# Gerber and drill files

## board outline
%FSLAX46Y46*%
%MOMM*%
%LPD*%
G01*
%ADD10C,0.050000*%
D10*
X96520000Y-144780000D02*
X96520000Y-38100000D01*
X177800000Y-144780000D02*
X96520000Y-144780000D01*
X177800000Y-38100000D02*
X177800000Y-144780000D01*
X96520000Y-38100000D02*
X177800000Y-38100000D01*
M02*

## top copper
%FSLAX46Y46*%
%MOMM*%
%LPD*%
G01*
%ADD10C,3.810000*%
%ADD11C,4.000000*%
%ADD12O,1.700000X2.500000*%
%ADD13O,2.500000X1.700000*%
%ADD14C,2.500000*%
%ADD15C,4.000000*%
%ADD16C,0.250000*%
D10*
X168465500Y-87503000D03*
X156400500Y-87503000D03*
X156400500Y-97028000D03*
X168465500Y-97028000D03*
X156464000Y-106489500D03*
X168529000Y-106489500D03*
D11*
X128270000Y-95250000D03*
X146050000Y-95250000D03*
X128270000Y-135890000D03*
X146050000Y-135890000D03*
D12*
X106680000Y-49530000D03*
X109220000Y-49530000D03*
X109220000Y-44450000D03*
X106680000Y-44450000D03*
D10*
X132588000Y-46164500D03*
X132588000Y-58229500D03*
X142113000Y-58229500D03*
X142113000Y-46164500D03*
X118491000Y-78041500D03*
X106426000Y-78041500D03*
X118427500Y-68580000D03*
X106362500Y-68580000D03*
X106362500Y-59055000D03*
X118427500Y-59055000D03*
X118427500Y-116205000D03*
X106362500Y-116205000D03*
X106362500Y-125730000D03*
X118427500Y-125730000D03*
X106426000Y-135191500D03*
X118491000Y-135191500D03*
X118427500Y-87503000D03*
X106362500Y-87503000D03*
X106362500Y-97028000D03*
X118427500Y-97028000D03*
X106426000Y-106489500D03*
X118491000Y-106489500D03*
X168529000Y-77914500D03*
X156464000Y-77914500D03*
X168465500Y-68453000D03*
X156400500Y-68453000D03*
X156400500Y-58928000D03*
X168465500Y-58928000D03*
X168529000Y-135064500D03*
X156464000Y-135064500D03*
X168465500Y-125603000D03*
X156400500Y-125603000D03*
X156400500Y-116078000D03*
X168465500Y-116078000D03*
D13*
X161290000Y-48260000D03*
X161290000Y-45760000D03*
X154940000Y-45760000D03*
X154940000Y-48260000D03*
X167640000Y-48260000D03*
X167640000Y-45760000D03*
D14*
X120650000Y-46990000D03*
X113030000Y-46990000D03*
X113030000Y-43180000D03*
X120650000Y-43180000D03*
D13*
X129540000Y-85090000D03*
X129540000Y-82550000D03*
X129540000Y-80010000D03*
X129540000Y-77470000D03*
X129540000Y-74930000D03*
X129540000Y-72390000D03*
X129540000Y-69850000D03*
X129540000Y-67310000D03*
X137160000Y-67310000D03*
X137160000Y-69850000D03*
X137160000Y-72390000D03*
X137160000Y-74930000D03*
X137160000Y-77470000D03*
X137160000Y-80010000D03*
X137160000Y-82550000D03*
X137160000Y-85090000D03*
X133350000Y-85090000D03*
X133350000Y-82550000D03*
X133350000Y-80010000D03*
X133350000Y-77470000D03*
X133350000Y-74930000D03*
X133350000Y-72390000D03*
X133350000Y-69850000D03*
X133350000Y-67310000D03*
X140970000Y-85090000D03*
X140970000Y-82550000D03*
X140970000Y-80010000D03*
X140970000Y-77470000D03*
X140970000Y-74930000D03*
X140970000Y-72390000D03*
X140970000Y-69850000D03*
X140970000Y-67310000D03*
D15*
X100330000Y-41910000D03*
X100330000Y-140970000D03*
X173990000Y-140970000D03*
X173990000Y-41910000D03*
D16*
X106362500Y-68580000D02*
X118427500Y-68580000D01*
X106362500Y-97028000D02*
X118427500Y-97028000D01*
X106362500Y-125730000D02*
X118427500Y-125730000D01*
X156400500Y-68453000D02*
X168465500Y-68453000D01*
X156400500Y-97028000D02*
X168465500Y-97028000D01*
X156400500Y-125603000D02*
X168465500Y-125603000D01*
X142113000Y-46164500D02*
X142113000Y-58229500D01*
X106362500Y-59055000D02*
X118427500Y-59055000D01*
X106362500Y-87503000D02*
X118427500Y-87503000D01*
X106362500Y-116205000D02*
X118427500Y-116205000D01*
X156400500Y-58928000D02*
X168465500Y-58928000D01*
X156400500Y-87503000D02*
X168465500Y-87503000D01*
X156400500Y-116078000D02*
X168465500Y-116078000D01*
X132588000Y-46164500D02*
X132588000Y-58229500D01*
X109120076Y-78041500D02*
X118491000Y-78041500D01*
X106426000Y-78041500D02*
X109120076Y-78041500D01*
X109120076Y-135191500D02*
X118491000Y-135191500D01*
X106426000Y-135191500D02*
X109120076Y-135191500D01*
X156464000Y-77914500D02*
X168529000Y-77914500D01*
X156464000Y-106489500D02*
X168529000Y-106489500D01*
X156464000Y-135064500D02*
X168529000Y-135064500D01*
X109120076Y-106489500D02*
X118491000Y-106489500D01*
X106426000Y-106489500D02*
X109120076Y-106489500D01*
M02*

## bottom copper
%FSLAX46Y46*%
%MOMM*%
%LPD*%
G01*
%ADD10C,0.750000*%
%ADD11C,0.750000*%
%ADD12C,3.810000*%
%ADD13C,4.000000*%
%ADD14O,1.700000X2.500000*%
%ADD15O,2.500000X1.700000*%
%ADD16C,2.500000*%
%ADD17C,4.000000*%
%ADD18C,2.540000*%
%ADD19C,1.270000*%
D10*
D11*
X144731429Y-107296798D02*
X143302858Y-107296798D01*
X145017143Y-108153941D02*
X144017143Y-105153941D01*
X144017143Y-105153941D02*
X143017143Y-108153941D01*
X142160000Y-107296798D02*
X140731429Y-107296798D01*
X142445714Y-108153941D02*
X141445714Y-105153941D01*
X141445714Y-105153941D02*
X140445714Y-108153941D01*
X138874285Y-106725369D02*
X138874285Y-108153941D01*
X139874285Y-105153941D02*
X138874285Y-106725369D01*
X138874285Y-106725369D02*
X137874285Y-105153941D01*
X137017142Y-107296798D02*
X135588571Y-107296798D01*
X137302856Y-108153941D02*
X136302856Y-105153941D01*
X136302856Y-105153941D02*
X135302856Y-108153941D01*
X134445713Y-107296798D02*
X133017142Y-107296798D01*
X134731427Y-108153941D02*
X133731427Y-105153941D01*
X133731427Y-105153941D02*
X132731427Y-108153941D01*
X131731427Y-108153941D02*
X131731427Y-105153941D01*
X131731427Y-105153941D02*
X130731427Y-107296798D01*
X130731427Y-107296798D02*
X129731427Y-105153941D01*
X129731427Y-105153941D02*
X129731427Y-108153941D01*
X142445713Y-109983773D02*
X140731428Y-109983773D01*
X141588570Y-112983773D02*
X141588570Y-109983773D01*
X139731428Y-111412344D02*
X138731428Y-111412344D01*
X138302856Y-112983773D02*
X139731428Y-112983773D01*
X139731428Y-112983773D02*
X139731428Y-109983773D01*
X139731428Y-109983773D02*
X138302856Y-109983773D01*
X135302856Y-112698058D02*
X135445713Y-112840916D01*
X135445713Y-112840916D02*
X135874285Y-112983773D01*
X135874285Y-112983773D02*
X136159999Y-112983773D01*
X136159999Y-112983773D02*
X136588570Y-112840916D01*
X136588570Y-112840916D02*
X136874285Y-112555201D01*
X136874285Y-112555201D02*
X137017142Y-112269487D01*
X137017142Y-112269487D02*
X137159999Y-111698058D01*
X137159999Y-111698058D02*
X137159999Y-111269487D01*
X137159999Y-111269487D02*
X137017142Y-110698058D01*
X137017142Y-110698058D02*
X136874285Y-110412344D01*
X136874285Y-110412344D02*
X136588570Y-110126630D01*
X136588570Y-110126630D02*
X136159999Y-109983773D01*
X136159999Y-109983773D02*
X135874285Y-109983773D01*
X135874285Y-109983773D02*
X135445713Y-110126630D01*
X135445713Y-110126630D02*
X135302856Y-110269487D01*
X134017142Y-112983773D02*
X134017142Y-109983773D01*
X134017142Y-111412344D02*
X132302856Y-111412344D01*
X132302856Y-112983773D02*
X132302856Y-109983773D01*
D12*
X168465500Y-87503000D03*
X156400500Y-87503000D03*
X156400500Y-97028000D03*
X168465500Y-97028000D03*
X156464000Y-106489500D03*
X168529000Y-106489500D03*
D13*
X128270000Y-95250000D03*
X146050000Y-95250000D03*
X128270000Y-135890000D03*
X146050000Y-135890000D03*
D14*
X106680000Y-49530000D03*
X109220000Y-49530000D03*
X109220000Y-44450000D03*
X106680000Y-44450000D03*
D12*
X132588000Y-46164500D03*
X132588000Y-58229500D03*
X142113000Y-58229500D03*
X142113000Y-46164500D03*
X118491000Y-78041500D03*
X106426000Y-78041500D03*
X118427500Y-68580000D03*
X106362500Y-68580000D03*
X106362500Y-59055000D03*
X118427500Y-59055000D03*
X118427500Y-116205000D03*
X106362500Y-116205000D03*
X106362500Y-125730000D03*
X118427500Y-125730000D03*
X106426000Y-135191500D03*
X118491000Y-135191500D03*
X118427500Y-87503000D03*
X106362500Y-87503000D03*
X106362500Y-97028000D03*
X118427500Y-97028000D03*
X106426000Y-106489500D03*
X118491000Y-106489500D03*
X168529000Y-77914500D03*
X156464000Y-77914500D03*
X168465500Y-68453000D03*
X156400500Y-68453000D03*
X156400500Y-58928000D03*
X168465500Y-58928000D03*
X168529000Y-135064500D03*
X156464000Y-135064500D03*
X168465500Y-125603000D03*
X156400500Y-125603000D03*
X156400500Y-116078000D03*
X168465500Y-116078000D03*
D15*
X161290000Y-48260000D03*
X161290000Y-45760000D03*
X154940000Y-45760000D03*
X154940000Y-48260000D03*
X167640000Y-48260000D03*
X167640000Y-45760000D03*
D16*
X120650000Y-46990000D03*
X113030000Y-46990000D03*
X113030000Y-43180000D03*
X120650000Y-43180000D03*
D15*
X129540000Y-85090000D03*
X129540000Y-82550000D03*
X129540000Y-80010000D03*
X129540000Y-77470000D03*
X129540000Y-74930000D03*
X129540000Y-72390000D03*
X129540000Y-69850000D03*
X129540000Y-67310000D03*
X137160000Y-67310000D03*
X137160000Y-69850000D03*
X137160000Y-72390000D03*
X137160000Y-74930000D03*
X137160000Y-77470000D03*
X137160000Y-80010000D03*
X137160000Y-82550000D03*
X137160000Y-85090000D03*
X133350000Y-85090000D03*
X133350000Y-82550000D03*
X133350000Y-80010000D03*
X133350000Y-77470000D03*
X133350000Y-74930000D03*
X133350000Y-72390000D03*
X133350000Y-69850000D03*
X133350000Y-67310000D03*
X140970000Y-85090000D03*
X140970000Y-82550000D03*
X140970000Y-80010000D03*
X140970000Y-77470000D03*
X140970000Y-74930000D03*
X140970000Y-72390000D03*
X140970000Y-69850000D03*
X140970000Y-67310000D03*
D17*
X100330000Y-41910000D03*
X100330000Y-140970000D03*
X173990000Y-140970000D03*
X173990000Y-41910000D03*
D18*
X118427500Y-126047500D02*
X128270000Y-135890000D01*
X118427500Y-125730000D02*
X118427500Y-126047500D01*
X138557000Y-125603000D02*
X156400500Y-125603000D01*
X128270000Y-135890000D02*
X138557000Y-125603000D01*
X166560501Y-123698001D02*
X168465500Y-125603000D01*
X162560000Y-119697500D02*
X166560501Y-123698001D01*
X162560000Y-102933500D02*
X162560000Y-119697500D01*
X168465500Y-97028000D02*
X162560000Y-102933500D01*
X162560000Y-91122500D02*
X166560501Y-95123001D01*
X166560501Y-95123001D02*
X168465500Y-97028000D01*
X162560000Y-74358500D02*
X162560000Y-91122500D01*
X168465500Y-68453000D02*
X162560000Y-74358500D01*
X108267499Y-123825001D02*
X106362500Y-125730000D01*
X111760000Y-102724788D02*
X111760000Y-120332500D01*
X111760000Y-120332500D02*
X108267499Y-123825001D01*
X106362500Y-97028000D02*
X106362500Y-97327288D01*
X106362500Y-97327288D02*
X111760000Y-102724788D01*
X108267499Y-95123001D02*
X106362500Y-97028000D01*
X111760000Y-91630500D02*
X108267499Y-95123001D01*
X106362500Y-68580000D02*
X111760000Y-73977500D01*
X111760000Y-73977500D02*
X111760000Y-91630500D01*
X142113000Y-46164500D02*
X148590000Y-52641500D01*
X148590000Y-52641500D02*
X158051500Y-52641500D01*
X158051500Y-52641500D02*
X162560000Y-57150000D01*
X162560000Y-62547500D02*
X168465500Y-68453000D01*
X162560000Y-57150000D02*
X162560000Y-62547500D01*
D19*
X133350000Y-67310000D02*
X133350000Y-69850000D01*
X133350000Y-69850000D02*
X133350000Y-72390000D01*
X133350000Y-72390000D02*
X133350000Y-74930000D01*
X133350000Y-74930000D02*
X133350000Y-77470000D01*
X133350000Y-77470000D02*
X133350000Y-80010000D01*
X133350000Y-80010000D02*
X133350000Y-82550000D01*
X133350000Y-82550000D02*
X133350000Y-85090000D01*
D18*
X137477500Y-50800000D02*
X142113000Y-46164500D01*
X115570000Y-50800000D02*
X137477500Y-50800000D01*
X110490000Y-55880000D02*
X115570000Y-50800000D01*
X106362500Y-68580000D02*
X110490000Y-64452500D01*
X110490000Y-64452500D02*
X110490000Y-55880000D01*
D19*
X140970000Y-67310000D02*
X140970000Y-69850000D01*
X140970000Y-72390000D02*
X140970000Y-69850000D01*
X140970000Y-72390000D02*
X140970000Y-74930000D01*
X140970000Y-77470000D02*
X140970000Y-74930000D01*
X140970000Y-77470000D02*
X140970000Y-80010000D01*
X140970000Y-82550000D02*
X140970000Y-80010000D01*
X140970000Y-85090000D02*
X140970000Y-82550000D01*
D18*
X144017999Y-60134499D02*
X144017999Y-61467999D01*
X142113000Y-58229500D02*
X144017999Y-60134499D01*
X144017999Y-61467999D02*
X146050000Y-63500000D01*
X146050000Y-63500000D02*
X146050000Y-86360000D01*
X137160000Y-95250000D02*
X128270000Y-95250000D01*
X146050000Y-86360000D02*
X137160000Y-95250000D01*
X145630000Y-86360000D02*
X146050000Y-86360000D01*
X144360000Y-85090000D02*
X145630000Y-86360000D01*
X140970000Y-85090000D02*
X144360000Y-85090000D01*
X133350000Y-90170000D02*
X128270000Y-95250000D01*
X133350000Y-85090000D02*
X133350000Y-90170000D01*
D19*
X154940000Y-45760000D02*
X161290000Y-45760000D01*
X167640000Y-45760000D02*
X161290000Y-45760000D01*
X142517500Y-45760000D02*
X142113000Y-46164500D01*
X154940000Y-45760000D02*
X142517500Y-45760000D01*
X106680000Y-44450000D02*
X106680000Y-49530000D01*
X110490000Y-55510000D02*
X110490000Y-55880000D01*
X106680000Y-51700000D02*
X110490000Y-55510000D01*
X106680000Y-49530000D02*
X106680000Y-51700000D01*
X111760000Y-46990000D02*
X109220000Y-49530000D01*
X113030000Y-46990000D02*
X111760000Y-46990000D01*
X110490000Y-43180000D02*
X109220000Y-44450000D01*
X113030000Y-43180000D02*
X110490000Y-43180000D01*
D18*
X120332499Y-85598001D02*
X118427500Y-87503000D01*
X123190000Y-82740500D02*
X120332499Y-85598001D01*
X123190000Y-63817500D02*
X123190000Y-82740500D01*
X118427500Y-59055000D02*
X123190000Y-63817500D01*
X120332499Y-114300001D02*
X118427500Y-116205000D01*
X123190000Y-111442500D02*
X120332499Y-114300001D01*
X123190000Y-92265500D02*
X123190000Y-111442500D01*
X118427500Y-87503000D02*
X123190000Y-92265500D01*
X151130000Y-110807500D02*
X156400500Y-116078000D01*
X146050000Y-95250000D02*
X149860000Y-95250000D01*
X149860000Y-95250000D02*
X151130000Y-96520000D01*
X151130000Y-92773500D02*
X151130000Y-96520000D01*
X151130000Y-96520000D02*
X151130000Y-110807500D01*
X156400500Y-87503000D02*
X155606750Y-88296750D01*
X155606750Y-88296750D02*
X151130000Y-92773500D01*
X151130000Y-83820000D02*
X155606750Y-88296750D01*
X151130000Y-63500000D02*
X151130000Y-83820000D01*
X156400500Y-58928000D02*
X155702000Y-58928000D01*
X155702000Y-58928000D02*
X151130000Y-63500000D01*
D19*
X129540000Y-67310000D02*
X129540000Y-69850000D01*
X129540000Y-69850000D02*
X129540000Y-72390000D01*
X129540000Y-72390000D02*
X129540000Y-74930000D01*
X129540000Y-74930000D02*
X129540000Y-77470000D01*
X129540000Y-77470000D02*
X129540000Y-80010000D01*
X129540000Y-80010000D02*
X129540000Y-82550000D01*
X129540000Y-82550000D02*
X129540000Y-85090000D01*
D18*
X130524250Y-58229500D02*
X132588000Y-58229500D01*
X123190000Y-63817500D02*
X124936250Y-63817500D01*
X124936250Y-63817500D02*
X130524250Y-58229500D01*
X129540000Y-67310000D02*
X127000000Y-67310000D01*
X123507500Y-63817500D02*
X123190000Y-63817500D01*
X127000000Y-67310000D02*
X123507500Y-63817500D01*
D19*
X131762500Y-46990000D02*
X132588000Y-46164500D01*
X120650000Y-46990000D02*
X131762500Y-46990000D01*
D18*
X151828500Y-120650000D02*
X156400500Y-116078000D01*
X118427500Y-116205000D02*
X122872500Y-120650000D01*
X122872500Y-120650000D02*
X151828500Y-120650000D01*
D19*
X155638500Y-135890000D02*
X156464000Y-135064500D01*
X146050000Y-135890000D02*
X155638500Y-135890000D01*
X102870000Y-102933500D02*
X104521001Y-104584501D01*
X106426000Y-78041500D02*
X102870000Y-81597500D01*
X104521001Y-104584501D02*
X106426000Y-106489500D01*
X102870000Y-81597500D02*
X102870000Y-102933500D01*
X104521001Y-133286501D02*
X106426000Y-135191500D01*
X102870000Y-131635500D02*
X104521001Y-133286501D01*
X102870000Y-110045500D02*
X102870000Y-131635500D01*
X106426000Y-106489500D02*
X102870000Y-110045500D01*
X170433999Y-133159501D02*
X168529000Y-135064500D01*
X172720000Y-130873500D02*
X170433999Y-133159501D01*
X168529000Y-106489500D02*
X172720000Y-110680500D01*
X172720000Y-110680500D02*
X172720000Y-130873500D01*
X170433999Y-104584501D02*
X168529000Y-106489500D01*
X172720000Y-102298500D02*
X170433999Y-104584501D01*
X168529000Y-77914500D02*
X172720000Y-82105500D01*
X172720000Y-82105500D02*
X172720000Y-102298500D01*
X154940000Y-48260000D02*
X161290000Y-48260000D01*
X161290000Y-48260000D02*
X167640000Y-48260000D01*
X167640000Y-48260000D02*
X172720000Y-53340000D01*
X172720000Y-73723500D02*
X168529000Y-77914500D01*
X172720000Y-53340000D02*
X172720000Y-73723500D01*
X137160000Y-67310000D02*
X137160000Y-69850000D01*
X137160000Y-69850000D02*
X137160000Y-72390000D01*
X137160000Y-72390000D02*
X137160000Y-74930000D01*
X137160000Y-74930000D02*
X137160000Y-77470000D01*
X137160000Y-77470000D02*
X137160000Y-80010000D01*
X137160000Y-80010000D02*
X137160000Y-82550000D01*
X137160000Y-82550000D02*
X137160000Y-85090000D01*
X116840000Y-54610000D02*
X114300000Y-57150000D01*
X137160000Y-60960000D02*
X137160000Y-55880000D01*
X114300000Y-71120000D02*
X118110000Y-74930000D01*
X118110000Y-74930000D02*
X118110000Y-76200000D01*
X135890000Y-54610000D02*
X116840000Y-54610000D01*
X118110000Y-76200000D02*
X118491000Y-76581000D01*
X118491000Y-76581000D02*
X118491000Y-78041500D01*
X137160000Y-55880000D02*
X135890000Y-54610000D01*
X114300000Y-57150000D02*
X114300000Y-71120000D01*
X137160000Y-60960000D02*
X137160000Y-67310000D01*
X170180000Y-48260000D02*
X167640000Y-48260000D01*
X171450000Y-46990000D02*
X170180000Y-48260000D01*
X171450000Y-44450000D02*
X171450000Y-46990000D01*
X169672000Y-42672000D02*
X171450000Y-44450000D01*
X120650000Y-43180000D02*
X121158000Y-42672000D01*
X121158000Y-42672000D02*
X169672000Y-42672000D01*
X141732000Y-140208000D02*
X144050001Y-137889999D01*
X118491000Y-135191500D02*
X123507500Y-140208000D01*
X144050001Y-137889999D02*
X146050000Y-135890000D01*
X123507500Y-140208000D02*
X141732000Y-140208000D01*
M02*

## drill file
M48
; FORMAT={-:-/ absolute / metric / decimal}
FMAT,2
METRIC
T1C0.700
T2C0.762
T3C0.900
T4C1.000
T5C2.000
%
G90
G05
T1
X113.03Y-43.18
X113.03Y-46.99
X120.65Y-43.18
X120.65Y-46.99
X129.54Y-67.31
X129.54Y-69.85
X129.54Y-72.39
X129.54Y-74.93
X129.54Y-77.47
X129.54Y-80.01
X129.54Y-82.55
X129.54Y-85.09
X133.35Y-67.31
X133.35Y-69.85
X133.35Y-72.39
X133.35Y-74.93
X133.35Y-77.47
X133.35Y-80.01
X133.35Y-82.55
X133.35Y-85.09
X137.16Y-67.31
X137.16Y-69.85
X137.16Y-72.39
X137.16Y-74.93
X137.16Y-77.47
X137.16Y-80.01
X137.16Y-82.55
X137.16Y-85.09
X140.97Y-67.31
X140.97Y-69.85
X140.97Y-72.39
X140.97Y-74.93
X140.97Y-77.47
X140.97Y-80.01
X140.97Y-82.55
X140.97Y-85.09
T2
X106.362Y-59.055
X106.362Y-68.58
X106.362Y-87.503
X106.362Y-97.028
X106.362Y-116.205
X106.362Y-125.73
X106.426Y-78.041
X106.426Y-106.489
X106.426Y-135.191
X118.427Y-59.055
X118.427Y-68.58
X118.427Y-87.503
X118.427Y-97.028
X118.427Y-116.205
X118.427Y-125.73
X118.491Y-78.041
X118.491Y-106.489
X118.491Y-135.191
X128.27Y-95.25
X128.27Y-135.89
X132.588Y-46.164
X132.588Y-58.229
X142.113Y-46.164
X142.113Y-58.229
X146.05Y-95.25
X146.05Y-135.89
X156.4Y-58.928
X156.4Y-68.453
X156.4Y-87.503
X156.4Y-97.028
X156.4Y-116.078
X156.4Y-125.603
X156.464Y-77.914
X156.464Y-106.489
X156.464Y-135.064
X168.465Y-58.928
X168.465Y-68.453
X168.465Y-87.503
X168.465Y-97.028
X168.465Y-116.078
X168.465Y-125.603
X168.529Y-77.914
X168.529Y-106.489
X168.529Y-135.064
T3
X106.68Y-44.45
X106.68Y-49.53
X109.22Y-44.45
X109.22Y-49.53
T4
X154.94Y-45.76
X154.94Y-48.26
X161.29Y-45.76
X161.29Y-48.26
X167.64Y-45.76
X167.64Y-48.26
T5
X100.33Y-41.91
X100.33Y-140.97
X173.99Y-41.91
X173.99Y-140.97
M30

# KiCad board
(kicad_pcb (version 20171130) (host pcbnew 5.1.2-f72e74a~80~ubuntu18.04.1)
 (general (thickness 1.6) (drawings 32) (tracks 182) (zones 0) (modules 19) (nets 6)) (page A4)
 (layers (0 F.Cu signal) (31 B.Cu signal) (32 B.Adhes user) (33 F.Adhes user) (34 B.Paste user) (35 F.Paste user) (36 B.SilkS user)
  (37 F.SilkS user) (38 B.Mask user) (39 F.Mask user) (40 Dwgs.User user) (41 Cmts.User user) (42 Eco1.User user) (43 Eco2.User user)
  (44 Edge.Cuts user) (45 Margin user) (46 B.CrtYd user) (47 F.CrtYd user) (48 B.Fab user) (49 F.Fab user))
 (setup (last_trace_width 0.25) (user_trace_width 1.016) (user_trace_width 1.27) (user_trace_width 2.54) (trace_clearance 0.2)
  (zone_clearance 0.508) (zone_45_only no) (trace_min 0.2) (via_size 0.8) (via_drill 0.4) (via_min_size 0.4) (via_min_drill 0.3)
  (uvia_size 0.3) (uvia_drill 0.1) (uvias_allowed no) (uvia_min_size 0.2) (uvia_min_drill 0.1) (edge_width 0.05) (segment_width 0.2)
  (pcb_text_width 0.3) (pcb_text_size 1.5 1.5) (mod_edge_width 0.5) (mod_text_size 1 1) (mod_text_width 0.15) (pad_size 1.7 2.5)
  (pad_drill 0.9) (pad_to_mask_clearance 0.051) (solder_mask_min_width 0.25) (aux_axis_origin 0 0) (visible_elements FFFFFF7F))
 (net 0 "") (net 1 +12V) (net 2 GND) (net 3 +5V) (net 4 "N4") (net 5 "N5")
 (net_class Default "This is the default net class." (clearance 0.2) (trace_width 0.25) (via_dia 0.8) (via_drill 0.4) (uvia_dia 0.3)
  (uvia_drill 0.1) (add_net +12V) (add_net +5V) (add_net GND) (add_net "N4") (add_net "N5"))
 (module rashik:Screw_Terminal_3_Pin (layer F.Cu) (at 162.56 97.155 270)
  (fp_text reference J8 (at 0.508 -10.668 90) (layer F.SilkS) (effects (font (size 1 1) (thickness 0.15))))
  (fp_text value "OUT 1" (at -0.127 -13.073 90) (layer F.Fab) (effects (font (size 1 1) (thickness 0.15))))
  (pad 1 thru_hole circle (at -9.652 -5.9055 270) (size 3.81 3.81) (drill 0.762) (layers *.Cu *.Mask) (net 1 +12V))
  (pad 1 thru_hole circle (at -9.652 6.1595 270) (size 3.81 3.81) (drill 0.762) (layers *.Cu *.Mask) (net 1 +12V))
  (pad 2 thru_hole circle (at -0.127 6.1595 270) (size 3.81 3.81) (drill 0.762) (layers *.Cu *.Mask) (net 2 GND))
  (pad 2 thru_hole circle (at -0.127 -5.9055 270) (size 3.81 3.81) (drill 0.762) (layers *.Cu *.Mask) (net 2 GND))
  (pad 3 thru_hole circle (at 9.3345 6.096 270) (size 3.81 3.81) (drill 0.762) (layers *.Cu *.Mask) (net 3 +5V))
  (pad 3 thru_hole circle (at 9.3345 -5.969 270) (size 3.81 3.81) (drill 0.762) (layers *.Cu *.Mask) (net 3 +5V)))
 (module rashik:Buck (layer F.Cu) (at 135.89 115.57)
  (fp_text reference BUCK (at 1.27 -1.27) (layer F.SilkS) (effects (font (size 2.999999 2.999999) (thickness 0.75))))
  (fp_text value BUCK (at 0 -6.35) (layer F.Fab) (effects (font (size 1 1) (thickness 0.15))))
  (pad 1 thru_hole circle (at -7.62 -20.32) (size 4 4) (drill 0.762) (layers *.Cu *.Mask) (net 2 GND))
  (pad 2 thru_hole circle (at 10.16 -20.32) (size 4 4) (drill 0.762) (layers *.Cu *.Mask) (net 1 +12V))
  (pad 3 thru_hole circle (at -7.62 20.32) (size 4 4) (drill 0.762) (layers *.Cu *.Mask) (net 2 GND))
  (pad 4 thru_hole circle (at 10.16 20.32) (size 4 4) (drill 0.762) (layers *.Cu *.Mask) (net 3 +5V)))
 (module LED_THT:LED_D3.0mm (layer F.Cu) (at 106.68 49.53)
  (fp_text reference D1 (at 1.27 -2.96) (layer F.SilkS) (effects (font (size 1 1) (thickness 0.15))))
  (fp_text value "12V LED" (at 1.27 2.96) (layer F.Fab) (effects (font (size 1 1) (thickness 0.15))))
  (pad 1 thru_hole oval (at 0 0) (size 1.7 2.5) (drill 0.9) (layers *.Cu *.Mask) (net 2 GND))
  (pad 2 thru_hole oval (at 2.54 0) (size 1.7 2.5) (drill 0.9) (layers *.Cu *.Mask) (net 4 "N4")))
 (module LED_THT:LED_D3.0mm (layer F.Cu) (at 106.68 44.45)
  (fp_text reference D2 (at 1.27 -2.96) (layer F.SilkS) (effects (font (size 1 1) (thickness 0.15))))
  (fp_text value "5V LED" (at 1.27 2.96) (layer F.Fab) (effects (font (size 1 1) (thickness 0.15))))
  (pad 2 thru_hole oval (at 2.54 0) (size 1.7 2.5) (drill 0.9) (layers *.Cu *.Mask) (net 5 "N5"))
  (pad 1 thru_hole oval (at 0 0) (size 1.7 2.5) (drill 0.9) (layers *.Cu *.Mask) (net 2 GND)))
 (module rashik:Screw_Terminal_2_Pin (layer F.Cu) (at 142.24 52.07)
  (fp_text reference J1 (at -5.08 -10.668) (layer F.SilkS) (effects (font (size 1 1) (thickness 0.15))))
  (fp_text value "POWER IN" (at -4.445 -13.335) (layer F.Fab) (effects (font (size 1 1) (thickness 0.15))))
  (pad 1 thru_hole circle (at -9.652 -5.9055) (size 3.81 3.81) (drill 0.762) (layers *.Cu *.Mask) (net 1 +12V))
  (pad 1 thru_hole circle (at -9.652 6.1595) (size 3.81 3.81) (drill 0.762) (layers *.Cu *.Mask) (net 1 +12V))
  (pad 2 thru_hole circle (at -0.127 6.1595) (size 3.81 3.81) (drill 0.762) (layers *.Cu *.Mask) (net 2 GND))
  (pad 2 thru_hole circle (at -0.127 -5.9055) (size 3.81 3.81) (drill 0.762) (layers *.Cu *.Mask) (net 2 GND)))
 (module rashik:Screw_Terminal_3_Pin (layer F.Cu) (at 112.522 68.707 270)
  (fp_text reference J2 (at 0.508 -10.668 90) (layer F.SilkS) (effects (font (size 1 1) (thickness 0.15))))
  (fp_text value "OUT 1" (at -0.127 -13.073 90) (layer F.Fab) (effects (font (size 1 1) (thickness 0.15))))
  (pad 3 thru_hole circle (at 9.3345 -5.969 270) (size 3.81 3.81) (drill 0.762) (layers *.Cu *.Mask) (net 3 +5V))
  (pad 3 thru_hole circle (at 9.3345 6.096 270) (size 3.81 3.81) (drill 0.762) (layers *.Cu *.Mask) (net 3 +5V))
  (pad 2 thru_hole circle (at -0.127 -5.9055 270) (size 3.81 3.81) (drill 0.762) (layers *.Cu *.Mask) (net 2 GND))
  (pad 2 thru_hole circle (at -0.127 6.1595 270) (size 3.81 3.81) (drill 0.762) (layers *.Cu *.Mask) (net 2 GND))
  (pad 1 thru_hole circle (at -9.652 6.1595 270) (size 3.81 3.81) (drill 0.762) (layers *.Cu *.Mask) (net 1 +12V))
  (pad 1 thru_hole circle (at -9.652 -5.9055 270) (size 3.81 3.81) (drill 0.762) (layers *.Cu *.Mask) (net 1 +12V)))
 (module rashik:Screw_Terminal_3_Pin (layer F.Cu) (at 112.522 125.857 270)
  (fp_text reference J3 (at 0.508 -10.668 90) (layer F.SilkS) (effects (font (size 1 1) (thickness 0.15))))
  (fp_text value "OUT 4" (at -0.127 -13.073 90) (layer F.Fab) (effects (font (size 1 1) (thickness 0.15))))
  (pad 1 thru_hole circle (at -9.652 -5.9055 270) (size 3.81 3.81) (drill 0.762) (layers *.Cu *.Mask) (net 1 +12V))
  (pad 1 thru_hole circle (at -9.652 6.1595 270) (size 3.81 3.81) (drill 0.762) (layers *.Cu *.Mask) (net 1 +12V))
  (pad 2 thru_hole circle (at -0.127 6.1595 270) (size 3.81 3.81) (drill 0.762) (layers *.Cu *.Mask) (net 2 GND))
  (pad 2 thru_hole circle (at -0.127 -5.9055 270) (size 3.81 3.81) (drill 0.762) (layers *.Cu *.Mask) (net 2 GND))
  (pad 3 thru_hole circle (at 9.3345 6.096 270) (size 3.81 3.81) (drill 0.762) (layers *.Cu *.Mask) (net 3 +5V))
  (pad 3 thru_hole circle (at 9.3345 -5.969 270) (size 3.81 3.81) (drill 0.762) (layers *.Cu *.Mask) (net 3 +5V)))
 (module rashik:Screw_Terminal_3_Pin (layer F.Cu) (at 112.522 97.155 270)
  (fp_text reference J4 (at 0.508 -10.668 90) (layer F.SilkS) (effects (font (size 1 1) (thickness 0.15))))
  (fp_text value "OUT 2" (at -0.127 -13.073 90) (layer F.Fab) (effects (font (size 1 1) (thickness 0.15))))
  (pad 1 thru_hole circle (at -9.652 -5.9055 270) (size 3.81 3.81) (drill 0.762) (layers *.Cu *.Mask) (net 1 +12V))
  (pad 1 thru_hole circle (at -9.652 6.1595 270) (size 3.81 3.81) (drill 0.762) (layers *.Cu *.Mask) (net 1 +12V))
  (pad 2 thru_hole circle (at -0.127 6.1595 270) (size 3.81 3.81) (drill 0.762) (layers *.Cu *.Mask) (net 2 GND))
  (pad 2 thru_hole circle (at -0.127 -5.9055 270) (size 3.81 3.81) (drill 0.762) (layers *.Cu *.Mask) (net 2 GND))
  (pad 3 thru_hole circle (at 9.3345 6.096 270) (size 3.81 3.81) (drill 0.762) (layers *.Cu *.Mask) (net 3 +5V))
  (pad 3 thru_hole circle (at 9.3345 -5.969 270) (size 3.81 3.81) (drill 0.762) (layers *.Cu *.Mask) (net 3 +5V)))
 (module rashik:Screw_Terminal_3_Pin (layer F.Cu) (at 162.56 68.58 270)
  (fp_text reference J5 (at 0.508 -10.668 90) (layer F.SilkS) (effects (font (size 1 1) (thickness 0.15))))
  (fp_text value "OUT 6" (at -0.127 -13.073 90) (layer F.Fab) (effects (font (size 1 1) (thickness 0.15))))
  (pad 3 thru_hole circle (at 9.3345 -5.969 270) (size 3.81 3.81) (drill 0.762) (layers *.Cu *.Mask) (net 3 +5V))
  (pad 3 thru_hole circle (at 9.3345 6.096 270) (size 3.81 3.81) (drill 0.762) (layers *.Cu *.Mask) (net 3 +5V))
  (pad 2 thru_hole circle (at -0.127 -5.9055 270) (size 3.81 3.81) (drill 0.762) (layers *.Cu *.Mask) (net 2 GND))
  (pad 2 thru_hole circle (at -0.127 6.1595 270) (size 3.81 3.81) (drill 0.762) (layers *.Cu *.Mask) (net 2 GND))
  (pad 1 thru_hole circle (at -9.652 6.1595 270) (size 3.81 3.81) (drill 0.762) (layers *.Cu *.Mask) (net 1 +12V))
  (pad 1 thru_hole circle (at -9.652 -5.9055 270) (size 3.81 3.81) (drill 0.762) (layers *.Cu *.Mask) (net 1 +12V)))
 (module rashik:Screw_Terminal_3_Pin (layer F.Cu) (at 162.56 125.73 270)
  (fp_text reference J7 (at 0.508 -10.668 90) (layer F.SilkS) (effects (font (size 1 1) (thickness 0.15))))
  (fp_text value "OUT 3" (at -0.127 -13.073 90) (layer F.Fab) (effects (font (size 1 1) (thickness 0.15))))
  (pad 3 thru_hole circle (at 9.3345 -5.969 270) (size 3.81 3.81) (drill 0.762) (layers *.Cu *.Mask) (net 3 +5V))
  (pad 3 thru_hole circle (at 9.3345 6.096 270) (size 3.81 3.81) (drill 0.762) (layers *.Cu *.Mask) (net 3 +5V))
  (pad 2 thru_hole circle (at -0.127 -5.9055 270) (size 3.81 3.81) (drill 0.762) (layers *.Cu *.Mask) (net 2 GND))
  (pad 2 thru_hole circle (at -0.127 6.1595 270) (size 3.81 3.81) (drill 0.762) (layers *.Cu *.Mask) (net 2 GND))
  (pad 1 thru_hole circle (at -9.652 6.1595 270) (size 3.81 3.81) (drill 0.762) (layers *.Cu *.Mask) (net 1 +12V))
  (pad 1 thru_hole circle (at -9.652 -5.9055 270) (size 3.81 3.81) (drill 0.762) (layers *.Cu *.Mask) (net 1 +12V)))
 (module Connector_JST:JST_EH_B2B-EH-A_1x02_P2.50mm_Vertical (layer F.Cu) (at 161.29 48.26 90)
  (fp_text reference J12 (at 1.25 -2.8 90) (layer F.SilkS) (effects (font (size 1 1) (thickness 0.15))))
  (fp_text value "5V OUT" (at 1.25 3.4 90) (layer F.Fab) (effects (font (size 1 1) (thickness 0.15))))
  (pad 1 thru_hole oval (at 0 0 90) (size 1.7 2.5) (drill 1) (layers *.Cu *.Mask) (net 3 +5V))
  (pad 2 thru_hole oval (at 2.5 0 90) (size 1.7 2.5) (drill 1) (layers *.Cu *.Mask) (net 2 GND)))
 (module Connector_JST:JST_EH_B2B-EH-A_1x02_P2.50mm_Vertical (layer F.Cu) (at 154.94 48.26 90)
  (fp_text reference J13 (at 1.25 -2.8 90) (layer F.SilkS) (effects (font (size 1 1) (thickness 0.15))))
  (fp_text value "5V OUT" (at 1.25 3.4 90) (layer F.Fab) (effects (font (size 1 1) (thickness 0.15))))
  (pad 2 thru_hole oval (at 2.5 0 90) (size 1.7 2.5) (drill 1) (layers *.Cu *.Mask) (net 2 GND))
  (pad 1 thru_hole oval (at 0 0 90) (size 1.7 2.5) (drill 1) (layers *.Cu *.Mask) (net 3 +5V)))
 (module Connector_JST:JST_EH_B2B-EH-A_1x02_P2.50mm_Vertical (layer F.Cu) (at 167.64 48.26 90)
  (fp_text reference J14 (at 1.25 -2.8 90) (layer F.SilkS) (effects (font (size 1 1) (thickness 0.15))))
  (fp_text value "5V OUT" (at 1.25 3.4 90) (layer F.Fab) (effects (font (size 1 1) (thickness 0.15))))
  (pad 1 thru_hole oval (at 0 0 90) (size 1.7 2.5) (drill 1) (layers *.Cu *.Mask) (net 3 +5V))
  (pad 2 thru_hole oval (at 2.5 0 90) (size 1.7 2.5) (drill 1) (layers *.Cu *.Mask) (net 2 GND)))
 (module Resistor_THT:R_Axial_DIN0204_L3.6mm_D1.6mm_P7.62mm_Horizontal (layer F.Cu) (at 113.03 46.99)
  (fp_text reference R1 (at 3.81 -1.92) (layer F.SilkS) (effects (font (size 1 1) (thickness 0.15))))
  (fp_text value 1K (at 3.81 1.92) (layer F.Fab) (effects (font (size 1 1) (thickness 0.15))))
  (pad 2 thru_hole circle (at 7.62 0) (size 2.5 2.5) (drill 0.7) (layers *.Cu *.Mask) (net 1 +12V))
  (pad 1 thru_hole circle (at 0 0) (size 2.5 2.5) (drill 0.7) (layers *.Cu *.Mask) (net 4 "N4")))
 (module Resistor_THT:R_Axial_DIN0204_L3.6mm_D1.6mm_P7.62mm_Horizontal (layer F.Cu) (at 113.03 43.18)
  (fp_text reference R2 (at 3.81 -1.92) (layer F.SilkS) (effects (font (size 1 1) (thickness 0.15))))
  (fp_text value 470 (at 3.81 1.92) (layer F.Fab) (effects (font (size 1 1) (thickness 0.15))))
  (pad 1 thru_hole circle (at 0 0) (size 2.5 2.5) (drill 0.7) (layers *.Cu *.Mask) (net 5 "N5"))
  (pad 2 thru_hole circle (at 7.62 0) (size 2.5 2.5) (drill 0.7) (layers *.Cu *.Mask) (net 3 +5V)))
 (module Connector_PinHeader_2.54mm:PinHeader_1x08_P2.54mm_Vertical (layer F.Cu) (at 129.54 85.09 180)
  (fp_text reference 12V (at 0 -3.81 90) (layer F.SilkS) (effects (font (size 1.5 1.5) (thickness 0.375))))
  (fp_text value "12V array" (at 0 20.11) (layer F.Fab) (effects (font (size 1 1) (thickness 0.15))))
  (pad 1 thru_hole oval (at 0 0 180) (size 2.5 1.7) (drill 0.7) (layers *.Cu *.Mask) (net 1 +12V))
  (pad 2 thru_hole oval (at 0 2.54 180) (size 2.5 1.7) (drill 0.7) (layers *.Cu *.Mask) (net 1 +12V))
  (pad 3 thru_hole oval (at 0 5.08 180) (size 2.5 1.7) (drill 0.7) (layers *.Cu *.Mask) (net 1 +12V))
  (pad 4 thru_hole oval (at 0 7.62 180) (size 2.5 1.7) (drill 0.7) (layers *.Cu *.Mask) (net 1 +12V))
  (pad 5 thru_hole oval (at 0 10.16 180) (size 2.5 1.7) (drill 0.7) (layers *.Cu *.Mask) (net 1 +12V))
  (pad 6 thru_hole oval (at 0 12.7 180) (size 2.5 1.7) (drill 0.7) (layers *.Cu *.Mask) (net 1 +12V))
  (pad 7 thru_hole oval (at 0 15.24 180) (size 2.5 1.7) (drill 0.7) (layers *.Cu *.Mask) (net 1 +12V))
  (pad 8 thru_hole oval (at 0 17.78 180) (size 2.5 1.7) (drill 0.7) (layers *.Cu *.Mask) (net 1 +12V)))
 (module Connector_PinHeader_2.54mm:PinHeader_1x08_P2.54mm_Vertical (layer F.Cu) (at 137.16 85.09 180)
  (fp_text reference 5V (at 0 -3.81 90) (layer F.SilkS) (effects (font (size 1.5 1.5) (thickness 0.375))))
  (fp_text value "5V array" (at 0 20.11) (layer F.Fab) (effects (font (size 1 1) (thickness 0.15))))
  (pad 8 thru_hole oval (at 0 17.78 180) (size 2.5 1.7) (drill 0.7) (layers *.Cu *.Mask) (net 3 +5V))
  (pad 7 thru_hole oval (at 0 15.24 180) (size 2.5 1.7) (drill 0.7) (layers *.Cu *.Mask) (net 3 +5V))
  (pad 6 thru_hole oval (at 0 12.7 180) (size 2.5 1.7) (drill 0.7) (layers *.Cu *.Mask) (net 3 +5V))
  (pad 5 thru_hole oval (at 0 10.16 180) (size 2.5 1.7) (drill 0.7) (layers *.Cu *.Mask) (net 3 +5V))
  (pad 4 thru_hole oval (at 0 7.62 180) (size 2.5 1.7) (drill 0.7) (layers *.Cu *.Mask) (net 3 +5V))
  (pad 3 thru_hole oval (at 0 5.08 180) (size 2.5 1.7) (drill 0.7) (layers *.Cu *.Mask) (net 3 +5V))
  (pad 2 thru_hole oval (at 0 2.54 180) (size 2.5 1.7) (drill 0.7) (layers *.Cu *.Mask) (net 3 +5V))
  (pad 1 thru_hole oval (at 0 0 180) (size 2.5 1.7) (drill 0.7) (layers *.Cu *.Mask) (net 3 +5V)))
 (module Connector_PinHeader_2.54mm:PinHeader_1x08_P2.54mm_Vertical (layer F.Cu) (at 133.35 85.09 180)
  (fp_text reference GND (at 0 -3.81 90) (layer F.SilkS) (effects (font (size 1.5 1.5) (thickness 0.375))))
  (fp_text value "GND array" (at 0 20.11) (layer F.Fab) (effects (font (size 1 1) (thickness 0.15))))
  (pad 1 thru_hole oval (at 0 0 180) (size 2.5 1.7) (drill 0.7) (layers *.Cu *.Mask) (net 2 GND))
  (pad 2 thru_hole oval (at 0 2.54 180) (size 2.5 1.7) (drill 0.7) (layers *.Cu *.Mask) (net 2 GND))
  (pad 3 thru_hole oval (at 0 5.08 180) (size 2.5 1.7) (drill 0.7) (layers *.Cu *.Mask) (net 2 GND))
  (pad 4 thru_hole oval (at 0 7.62 180) (size 2.5 1.7) (drill 0.7) (layers *.Cu *.Mask) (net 2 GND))
  (pad 5 thru_hole oval (at 0 10.16 180) (size 2.5 1.7) (drill 0.7) (layers *.Cu *.Mask) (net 2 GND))
  (pad 6 thru_hole oval (at 0 12.7 180) (size 2.5 1.7) (drill 0.7) (layers *.Cu *.Mask) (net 2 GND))
  (pad 7 thru_hole oval (at 0 15.24 180) (size 2.5 1.7) (drill 0.7) (layers *.Cu *.Mask) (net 2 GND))
  (pad 8 thru_hole oval (at 0 17.78 180) (size 2.5 1.7) (drill 0.7) (layers *.Cu *.Mask) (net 2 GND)))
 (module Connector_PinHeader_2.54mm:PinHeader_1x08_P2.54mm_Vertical (layer F.Cu) (at 140.97 85.09 180)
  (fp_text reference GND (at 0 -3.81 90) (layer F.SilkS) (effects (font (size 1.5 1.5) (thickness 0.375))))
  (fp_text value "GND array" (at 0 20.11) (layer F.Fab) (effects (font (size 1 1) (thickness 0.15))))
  (pad 1 thru_hole oval (at 0 0 180) (size 2.5 1.7) (drill 0.7) (layers *.Cu *.Mask) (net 2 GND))
  (pad 2 thru_hole oval (at 0 2.54 180) (size 2.5 1.7) (drill 0.7) (layers *.Cu *.Mask) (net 2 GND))
  (pad 3 thru_hole oval (at 0 5.08 180) (size 2.5 1.7) (drill 0.7) (layers *.Cu *.Mask) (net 2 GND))
  (pad 4 thru_hole oval (at 0 7.62 180) (size 2.5 1.7) (drill 0.7) (layers *.Cu *.Mask) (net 2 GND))
  (pad 5 thru_hole oval (at 0 10.16 180) (size 2.5 1.7) (drill 0.7) (layers *.Cu *.Mask) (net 2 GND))
  (pad 6 thru_hole oval (at 0 12.7 180) (size 2.5 1.7) (drill 0.7) (layers *.Cu *.Mask) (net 2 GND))
  (pad 7 thru_hole oval (at 0 15.24 180) (size 2.5 1.7) (drill 0.7) (layers *.Cu *.Mask) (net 2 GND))
  (pad 8 thru_hole oval (at 0 17.78 180) (size 2.5 1.7) (drill 0.7) (layers *.Cu *.Mask) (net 2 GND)))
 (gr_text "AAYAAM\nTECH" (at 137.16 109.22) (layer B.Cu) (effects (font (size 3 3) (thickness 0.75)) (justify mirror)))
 (gr_line (start 96.52 144.78) (end 96.52 38.1) (layer Edge.Cuts) (width 0.05))
 (gr_line (start 177.8 144.78) (end 96.52 144.78) (layer Edge.Cuts) (width 0.05))
 (gr_line (start 177.8 38.1) (end 177.8 144.78) (layer Edge.Cuts) (width 0.05))
 (gr_line (start 96.52 38.1) (end 177.8 38.1) (layer Edge.Cuts) (width 0.05))
 (via (at 100.33 41.91) (size 4) (drill 2) (layers F.Cu B.Cu) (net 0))
 (via (at 100.33 140.97) (size 4) (drill 2) (layers F.Cu B.Cu) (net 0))
 (via (at 173.99 140.97) (size 4) (drill 2) (layers F.Cu B.Cu) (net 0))
 (via (at 173.99 41.91) (size 4) (drill 2) (layers F.Cu B.Cu) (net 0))
 (segment (start 118.4275 126.0475) (end 128.27 135.89) (width 2.54) (layer B.Cu) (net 2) (status 30))
 (segment (start 118.4275 125.73) (end 118.4275 126.0475) (width 2.54) (layer B.Cu) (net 2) (status 30))
 (segment (start 138.557 125.603) (end 156.4005 125.603) (width 2.54) (layer B.Cu) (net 2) (status 20))
 (segment (start 128.27 135.89) (end 138.557 125.603) (width 2.54) (layer B.Cu) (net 2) (status 10))
 (segment (start 166.560501 123.698001) (end 168.4655 125.603) (width 2.54) (layer B.Cu) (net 2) (status 20))
 (segment (start 162.56 119.6975) (end 166.560501 123.698001) (width 2.54) (layer B.Cu) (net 2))
 (segment (start 162.56 102.9335) (end 162.56 119.6975) (width 2.54) (layer B.Cu) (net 2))
 (segment (start 168.4655 97.028) (end 162.56 102.9335) (width 2.54) (layer B.Cu) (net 2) (status 10))
 (segment (start 162.56 91.1225) (end 166.560501 95.123001) (width 2.54) (layer B.Cu) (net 2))
 (segment (start 166.560501 95.123001) (end 168.4655 97.028) (width 2.54) (layer B.Cu) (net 2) (status 20))
 (segment (start 162.56 74.3585) (end 162.56 91.1225) (width 2.54) (layer B.Cu) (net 2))
 (segment (start 168.4655 68.453) (end 162.56 74.3585) (width 2.54) (layer B.Cu) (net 2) (status 10))
 (segment (start 108.267499 123.825001) (end 106.3625 125.73) (width 2.54) (layer B.Cu) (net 2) (status 20))
 (segment (start 111.76 102.724788) (end 111.76 120.3325) (width 2.54) (layer B.Cu) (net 2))
 (segment (start 111.76 120.3325) (end 108.267499 123.825001) (width 2.54) (layer B.Cu) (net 2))
 (segment (start 106.3625 97.028) (end 106.3625 97.327288) (width 2.54) (layer B.Cu) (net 2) (status 30))
 (segment (start 106.3625 97.327288) (end 111.76 102.724788) (width 2.54) (layer B.Cu) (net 2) (status 10))
 (segment (start 108.267499 95.123001) (end 106.3625 97.028) (width 2.54) (layer B.Cu) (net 2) (status 20))
 (segment (start 111.76 91.6305) (end 108.267499 95.123001) (width 2.54) (layer B.Cu) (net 2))
 (segment (start 106.3625 68.58) (end 111.76 73.9775) (width 2.54) (layer B.Cu) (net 2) (status 10))
 (segment (start 111.76 73.9775) (end 111.76 91.6305) (width 2.54) (layer B.Cu) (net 2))
 (segment (start 142.113 46.1645) (end 148.59 52.6415) (width 2.54) (layer B.Cu) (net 2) (status 10))
 (segment (start 148.59 52.6415) (end 158.0515 52.6415) (width 2.54) (layer B.Cu) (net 2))
 (segment (start 158.0515 52.6415) (end 162.56 57.15) (width 2.54) (layer B.Cu) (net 2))
 (segment (start 162.56 62.5475) (end 168.4655 68.453) (width 2.54) (layer B.Cu) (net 2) (status 20))
 (segment (start 162.56 57.15) (end 162.56 62.5475) (width 2.54) (layer B.Cu) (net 2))
 (segment (start 133.35 67.31) (end 133.35 69.85) (width 1.27) (layer B.Cu) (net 2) (status 30))
 (segment (start 133.35 69.85) (end 133.35 72.39) (width 1.27) (layer B.Cu) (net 2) (status 30))
 (segment (start 133.35 72.39) (end 133.35 74.93) (width 1.27) (layer B.Cu) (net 2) (status 30))
 (segment (start 133.35 74.93) (end 133.35 77.47) (width 1.27) (layer B.Cu) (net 2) (status 30))
 (segment (start 133.35 77.47) (end 133.35 80.01) (width 1.27) (layer B.Cu) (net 2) (status 30))
 (segment (start 133.35 80.01) (end 133.35 82.55) (width 1.27) (layer B.Cu) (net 2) (status 30))
 (segment (start 133.35 82.55) (end 133.35 85.09) (width 1.27) (layer B.Cu) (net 2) (status 30))
 (segment (start 137.4775 50.8) (end 142.113 46.1645) (width 2.54) (layer B.Cu) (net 2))
 (segment (start 115.57 50.8) (end 137.4775 50.8) (width 2.54) (layer B.Cu) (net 2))
 (segment (start 110.49 55.88) (end 115.57 50.8) (width 2.54) (layer B.Cu) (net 2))
 (segment (start 106.3625 68.58) (end 110.49 64.4525) (width 2.54) (layer B.Cu) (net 2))
 (segment (start 110.49 64.4525) (end 110.49 55.88) (width 2.54) (layer B.Cu) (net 2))
 (segment (start 140.97 67.31) (end 140.97 69.85) (width 1.27) (layer B.Cu) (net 2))
 (segment (start 140.97 72.39) (end 140.97 69.85) (width 1.27) (layer B.Cu) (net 2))
 (segment (start 140.97 72.39) (end 140.97 74.93) (width 1.27) (layer B.Cu) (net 2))
 (segment (start 140.97 77.47) (end 140.97 74.93) (width 1.27) (layer B.Cu) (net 2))
 (segment (start 140.97 77.47) (end 140.97 80.01) (width 1.27) (layer B.Cu) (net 2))
 (segment (start 140.97 82.55) (end 140.97 80.01) (width 1.27) (layer B.Cu) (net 2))
 (segment (start 140.97 85.09) (end 140.97 82.55) (width 1.27) (layer B.Cu) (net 2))
 (segment (start 106.3625 68.58) (end 118.4275 68.58) (width 0.25) (layer F.Cu) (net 2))
 (segment (start 106.3625 97.028) (end 118.4275 97.028) (width 0.25) (layer F.Cu) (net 2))
 (segment (start 106.3625 125.73) (end 118.4275 125.73) (width 0.25) (layer F.Cu) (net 2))
 (segment (start 156.4005 68.453) (end 168.4655 68.453) (width 0.25) (layer F.Cu) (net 2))
 (segment (start 156.4005 97.028) (end 168.4655 97.028) (width 0.25) (layer F.Cu) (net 2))
 (segment (start 156.4005 125.603) (end 168.4655 125.603) (width 0.25) (layer F.Cu) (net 2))
 (segment (start 144.017999 60.134499) (end 144.017999 61.467999) (width 2.54) (layer B.Cu) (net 2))
 (segment (start 142.113 58.2295) (end 144.017999 60.134499) (width 2.54) (layer B.Cu) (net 2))
 (segment (start 144.017999 61.467999) (end 146.05 63.5) (width 2.54) (layer B.Cu) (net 2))
 (segment (start 146.05 63.5) (end 146.05 86.36) (width 2.54) (layer B.Cu) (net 2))
 (segment (start 137.16 95.25) (end 128.27 95.25) (width 2.54) (layer B.Cu) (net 2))
 (segment (start 146.05 86.36) (end 137.16 95.25) (width 2.54) (layer B.Cu) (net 2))
 (segment (start 145.63 86.36) (end 146.05 86.36) (width 2.54) (layer B.Cu) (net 2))
 (segment (start 144.36 85.09) (end 145.63 86.36) (width 2.54) (layer B.Cu) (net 2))
 (segment (start 140.97 85.09) (end 144.36 85.09) (width 2.54) (layer B.Cu) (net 2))
 (segment (start 133.35 90.17) (end 128.27 95.25) (width 2.54) (layer B.Cu) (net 2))
 (segment (start 133.35 85.09) (end 133.35 90.17) (width 2.54) (layer B.Cu) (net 2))
 (segment (start 154.94 45.76) (end 161.29 45.76) (width 1.27) (layer B.Cu) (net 2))
 (segment (start 167.64 45.76) (end 161.29 45.76) (width 1.27) (layer B.Cu) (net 2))
 (segment (start 142.5175 45.76) (end 142.113 46.1645) (width 1.27) (layer B.Cu) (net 2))
 (segment (start 154.94 45.76) (end 142.5175 45.76) (width 1.27) (layer B.Cu) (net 2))
 (segment (start 106.68 44.45) (end 106.68 49.53) (width 1.27) (layer B.Cu) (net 2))
 (segment (start 110.49 55.51) (end 110.49 55.88) (width 1.27) (layer B.Cu) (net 2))
 (segment (start 106.68 51.7) (end 110.49 55.51) (width 1.27) (layer B.Cu) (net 2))
 (segment (start 106.68 49.53) (end 106.68 51.7) (width 1.27) (layer B.Cu) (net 2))
 (segment (start 142.113 46.1645) (end 142.113 58.2295) (width 0.25) (layer F.Cu) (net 2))
 (segment (start 111.76 46.99) (end 109.22 49.53) (width 1.27) (layer B.Cu) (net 4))
 (segment (start 113.03 46.99) (end 111.76 46.99) (width 1.27) (layer B.Cu) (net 4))
 (segment (start 110.49 43.18) (end 109.22 44.45) (width 1.27) (layer B.Cu) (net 5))
 (segment (start 113.03 43.18) (end 110.49 43.18) (width 1.27) (layer B.Cu) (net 5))
 (segment (start 120.332499 85.598001) (end 118.4275 87.503) (width 2.54) (layer B.Cu) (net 1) (status 20))
 (segment (start 123.19 82.7405) (end 120.332499 85.598001) (width 2.54) (layer B.Cu) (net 1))
 (segment (start 123.19 63.8175) (end 123.19 82.7405) (width 2.54) (layer B.Cu) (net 1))
 (segment (start 118.4275 59.055) (end 123.19 63.8175) (width 2.54) (layer B.Cu) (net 1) (status 10))
 (segment (start 120.332499 114.300001) (end 118.4275 116.205) (width 2.54) (layer B.Cu) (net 1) (status 20))
 (segment (start 123.19 111.4425) (end 120.332499 114.300001) (width 2.54) (layer B.Cu) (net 1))
 (segment (start 123.19 92.2655) (end 123.19 111.4425) (width 2.54) (layer B.Cu) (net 1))
 (segment (start 118.4275 87.503) (end 123.19 92.2655) (width 2.54) (layer B.Cu) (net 1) (status 10))
 (segment (start 151.13 110.8075) (end 156.4005 116.078) (width 2.54) (layer B.Cu) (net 1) (status 20))
 (segment (start 146.05 95.25) (end 149.86 95.25) (width 2.54) (layer B.Cu) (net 1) (status 10))
 (segment (start 149.86 95.25) (end 151.13 96.52) (width 2.54) (layer B.Cu) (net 1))
 (segment (start 151.13 92.7735) (end 151.13 96.52) (width 2.54) (layer B.Cu) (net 1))
 (segment (start 151.13 96.52) (end 151.13 110.8075) (width 2.54) (layer B.Cu) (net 1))
 (segment (start 156.4005 87.503) (end 155.60675 88.29675) (width 2.54) (layer B.Cu) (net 1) (status 30))
 (segment (start 155.60675 88.29675) (end 151.13 92.7735) (width 2.54) (layer B.Cu) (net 1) (status 10))
 (segment (start 151.13 83.82) (end 155.60675 88.29675) (width 2.54) (layer B.Cu) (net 1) (status 20))
 (segment (start 151.13 63.5) (end 151.13 83.82) (width 2.54) (layer B.Cu) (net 1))
 (segment (start 156.4005 58.928) (end 155.702 58.928) (width 2.54) (layer B.Cu) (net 1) (status 30))
 (segment (start 155.702 58.928) (end 151.13 63.5) (width 2.54) (layer B.Cu) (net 1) (status 10))
 (segment (start 129.54 67.31) (end 129.54 69.85) (width 1.27) (layer B.Cu) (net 1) (status 30))
 (segment (start 129.54 69.85) (end 129.54 72.39) (width 1.27) (layer B.Cu) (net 1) (status 30))
 (segment (start 129.54 72.39) (end 129.54 74.93) (width 1.27) (layer B.Cu) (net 1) (status 30))
 (segment (start 129.54 74.93) (end 129.54 77.47) (width 1.27) (layer B.Cu) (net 1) (status 30))
 (segment (start 129.54 77.47) (end 129.54 80.01) (width 1.27) (layer B.Cu) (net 1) (status 30))
 (segment (start 129.54 80.01) (end 129.54 82.55) (width 1.27) (layer B.Cu) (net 1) (status 30))
 (segment (start 129.54 82.55) (end 129.54 85.09) (width 1.27) (layer B.Cu) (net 1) (status 30))
 (segment (start 130.52425 58.2295) (end 132.588 58.2295) (width 2.54) (layer B.Cu) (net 1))
 (segment (start 123.19 63.8175) (end 124.93625 63.8175) (width 2.54) (layer B.Cu) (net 1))
 (segment (start 124.93625 63.8175) (end 130.52425 58.2295) (width 2.54) (layer B.Cu) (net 1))
 (segment (start 106.3625 59.055) (end 118.4275 59.055) (width 0.25) (layer F.Cu) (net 1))
 (segment (start 106.3625 87.503) (end 118.4275 87.503) (width 0.25) (layer F.Cu) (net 1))
 (segment (start 106.3625 116.205) (end 118.4275 116.205) (width 0.25) (layer F.Cu) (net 1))
 (segment (start 156.4005 58.928) (end 168.4655 58.928) (width 0.25) (layer F.Cu) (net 1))
 (segment (start 156.4005 87.503) (end 168.4655 87.503) (width 0.25) (layer F.Cu) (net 1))
 (segment (start 156.4005 116.078) (end 168.4655 116.078) (width 0.25) (layer F.Cu) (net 1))
 (segment (start 129.54 67.31) (end 127 67.31) (width 2.54) (layer B.Cu) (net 1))
 (segment (start 123.5075 63.8175) (end 123.19 63.8175) (width 2.54) (layer B.Cu) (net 1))
 (segment (start 127 67.31) (end 123.5075 63.8175) (width 2.54) (layer B.Cu) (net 1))
 (segment (start 131.7625 46.99) (end 132.588 46.1645) (width 1.27) (layer B.Cu) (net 1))
 (segment (start 120.65 46.99) (end 131.7625 46.99) (width 1.27) (layer B.Cu) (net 1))
 (segment (start 132.588 46.1645) (end 132.588 58.2295) (width 0.25) (layer F.Cu) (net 1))
 (segment (start 151.8285 120.65) (end 156.4005 116.078) (width 2.54) (layer B.Cu) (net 1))
 (segment (start 118.4275 116.205) (end 122.8725 120.65) (width 2.54) (layer B.Cu) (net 1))
 (segment (start 122.8725 120.65) (end 151.8285 120.65) (width 2.54) (layer B.Cu) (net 1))
 (segment (start 155.6385 135.89) (end 156.464 135.0645) (width 1.27) (layer B.Cu) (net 3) (status 30))
 (segment (start 146.05 135.89) (end 155.6385 135.89) (width 1.27) (layer B.Cu) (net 3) (status 30))
 (segment (start 102.87 102.9335) (end 104.521001 104.584501) (width 1.27) (layer B.Cu) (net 3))
 (segment (start 106.426 78.0415) (end 102.87 81.5975) (width 1.27) (layer B.Cu) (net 3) (status 10))
 (segment (start 104.521001 104.584501) (end 106.426 106.4895) (width 1.27) (layer B.Cu) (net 3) (status 20))
 (segment (start 102.87 81.5975) (end 102.87 102.9335) (width 1.27) (layer B.Cu) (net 3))
 (segment (start 104.521001 133.286501) (end 106.426 135.1915) (width 1.27) (layer B.Cu) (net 3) (status 20))
 (segment (start 102.87 131.6355) (end 104.521001 133.286501) (width 1.27) (layer B.Cu) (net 3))
 (segment (start 102.87 110.0455) (end 102.87 131.6355) (width 1.27) (layer B.Cu) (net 3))
 (segment (start 106.426 106.4895) (end 102.87 110.0455) (width 1.27) (layer B.Cu) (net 3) (status 10))
 (segment (start 170.433999 133.159501) (end 168.529 135.0645) (width 1.27) (layer B.Cu) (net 3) (status 20))
 (segment (start 172.72 130.8735) (end 170.433999 133.159501) (width 1.27) (layer B.Cu) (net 3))
 (segment (start 168.529 106.4895) (end 172.72 110.6805) (width 1.27) (layer B.Cu) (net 3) (status 10))
 (segment (start 172.72 110.6805) (end 172.72 130.8735) (width 1.27) (layer B.Cu) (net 3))
 (segment (start 170.433999 104.584501) (end 168.529 106.4895) (width 1.27) (layer B.Cu) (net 3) (status 20))
 (segment (start 172.72 102.2985) (end 170.433999 104.584501) (width 1.27) (layer B.Cu) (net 3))
 (segment (start 168.529 77.9145) (end 172.72 82.1055) (width 1.27) (layer B.Cu) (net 3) (status 10))
 (segment (start 172.72 82.1055) (end 172.72 102.2985) (width 1.27) (layer B.Cu) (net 3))
 (segment (start 154.94 48.26) (end 161.29 48.26) (width 1.27) (layer B.Cu) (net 3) (status 30))
 (segment (start 161.29 48.26) (end 167.64 48.26) (width 1.27) (layer B.Cu) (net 3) (status 30))
 (segment (start 167.64 48.26) (end 172.72 53.34) (width 1.27) (layer B.Cu) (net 3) (status 10))
 (segment (start 172.72 73.7235) (end 168.529 77.9145) (width 1.27) (layer B.Cu) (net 3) (status 20))
 (segment (start 172.72 53.34) (end 172.72 73.7235) (width 1.27) (layer B.Cu) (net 3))
 (segment (start 137.16 67.31) (end 137.16 69.85) (width 1.27) (layer B.Cu) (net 3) (status 30))
 (segment (start 137.16 69.85) (end 137.16 72.39) (width 1.27) (layer B.Cu) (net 3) (status 30))
 (segment (start 137.16 72.39) (end 137.16 74.93) (width 1.27) (layer B.Cu) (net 3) (status 30))
 (segment (start 137.16 74.93) (end 137.16 77.47) (width 1.27) (layer B.Cu) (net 3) (status 30))
 (segment (start 137.16 77.47) (end 137.16 80.01) (width 1.27) (layer B.Cu) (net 3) (status 30))
 (segment (start 137.16 80.01) (end 137.16 82.55) (width 1.27) (layer B.Cu) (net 3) (status 30))
 (segment (start 137.16 82.55) (end 137.16 85.09) (width 1.27) (layer B.Cu) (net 3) (status 30))
 (segment (start 109.120076 78.0415) (end 118.491 78.0415) (width 0.25) (layer F.Cu) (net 3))
 (segment (start 106.426 78.0415) (end 109.120076 78.0415) (width 0.25) (layer F.Cu) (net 3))
 (segment (start 109.120076 135.1915) (end 118.491 135.1915) (width 0.25) (layer F.Cu) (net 3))
 (segment (start 106.426 135.1915) (end 109.120076 135.1915) (width 0.25) (layer F.Cu) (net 3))
 (segment (start 156.464 77.9145) (end 168.529 77.9145) (width 0.25) (layer F.Cu) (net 3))
 (segment (start 156.464 106.4895) (end 168.529 106.4895) (width 0.25) (layer F.Cu) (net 3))
 (segment (start 156.464 135.0645) (end 168.529 135.0645) (width 0.25) (layer F.Cu) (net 3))
 (segment (start 116.84 54.61) (end 114.3 57.15) (width 1.27) (layer B.Cu) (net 3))
 (segment (start 137.16 60.96) (end 137.16 55.88) (width 1.27) (layer B.Cu) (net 3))
 (segment (start 114.3 71.12) (end 118.11 74.93) (width 1.27) (layer B.Cu) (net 3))
 (segment (start 118.11 74.93) (end 118.11 76.2) (width 1.27) (layer B.Cu) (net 3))
 (segment (start 135.89 54.61) (end 116.84 54.61) (width 1.27) (layer B.Cu) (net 3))
 (segment (start 118.11 76.2) (end 118.491 76.581) (width 1.27) (layer B.Cu) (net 3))
 (segment (start 118.491 76.581) (end 118.491 78.0415) (width 1.27) (layer B.Cu) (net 3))
 (segment (start 137.16 55.88) (end 135.89 54.61) (width 1.27) (layer B.Cu) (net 3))
 (segment (start 114.3 57.15) (end 114.3 71.12) (width 1.27) (layer B.Cu) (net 3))
 (segment (start 137.16 60.96) (end 137.16 67.31) (width 1.27) (layer B.Cu) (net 3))
 (segment (start 170.18 48.26) (end 167.64 48.26) (width 1.27) (layer B.Cu) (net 3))
 (segment (start 171.45 46.99) (end 170.18 48.26) (width 1.27) (layer B.Cu) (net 3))
 (segment (start 171.45 44.45) (end 171.45 46.99) (width 1.27) (layer B.Cu) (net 3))
 (segment (start 169.672 42.672) (end 171.45 44.45) (width 1.27) (layer B.Cu) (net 3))
 (segment (start 120.65 43.18) (end 121.158 42.672) (width 1.27) (layer B.Cu) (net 3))
 (segment (start 121.158 42.672) (end 169.672 42.672) (width 1.27) (layer B.Cu) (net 3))
 (segment (start 109.120076 106.4895) (end 118.491 106.4895) (width 0.25) (layer F.Cu) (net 3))
 (segment (start 106.426 106.4895) (end 109.120076 106.4895) (width 0.25) (layer F.Cu) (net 3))
 (segment (start 141.732 140.208) (end 144.050001 137.889999) (width 1.27) (layer B.Cu) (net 3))
 (segment (start 118.491 135.1915) (end 123.5075 140.208) (width 1.27) (layer B.Cu) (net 3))
 (segment (start 144.050001 137.889999) (end 146.05 135.89) (width 1.27) (layer B.Cu) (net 3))
 (segment (start 123.5075 140.208) (end 141.732 140.208) (width 1.27) (layer B.Cu) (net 3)))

